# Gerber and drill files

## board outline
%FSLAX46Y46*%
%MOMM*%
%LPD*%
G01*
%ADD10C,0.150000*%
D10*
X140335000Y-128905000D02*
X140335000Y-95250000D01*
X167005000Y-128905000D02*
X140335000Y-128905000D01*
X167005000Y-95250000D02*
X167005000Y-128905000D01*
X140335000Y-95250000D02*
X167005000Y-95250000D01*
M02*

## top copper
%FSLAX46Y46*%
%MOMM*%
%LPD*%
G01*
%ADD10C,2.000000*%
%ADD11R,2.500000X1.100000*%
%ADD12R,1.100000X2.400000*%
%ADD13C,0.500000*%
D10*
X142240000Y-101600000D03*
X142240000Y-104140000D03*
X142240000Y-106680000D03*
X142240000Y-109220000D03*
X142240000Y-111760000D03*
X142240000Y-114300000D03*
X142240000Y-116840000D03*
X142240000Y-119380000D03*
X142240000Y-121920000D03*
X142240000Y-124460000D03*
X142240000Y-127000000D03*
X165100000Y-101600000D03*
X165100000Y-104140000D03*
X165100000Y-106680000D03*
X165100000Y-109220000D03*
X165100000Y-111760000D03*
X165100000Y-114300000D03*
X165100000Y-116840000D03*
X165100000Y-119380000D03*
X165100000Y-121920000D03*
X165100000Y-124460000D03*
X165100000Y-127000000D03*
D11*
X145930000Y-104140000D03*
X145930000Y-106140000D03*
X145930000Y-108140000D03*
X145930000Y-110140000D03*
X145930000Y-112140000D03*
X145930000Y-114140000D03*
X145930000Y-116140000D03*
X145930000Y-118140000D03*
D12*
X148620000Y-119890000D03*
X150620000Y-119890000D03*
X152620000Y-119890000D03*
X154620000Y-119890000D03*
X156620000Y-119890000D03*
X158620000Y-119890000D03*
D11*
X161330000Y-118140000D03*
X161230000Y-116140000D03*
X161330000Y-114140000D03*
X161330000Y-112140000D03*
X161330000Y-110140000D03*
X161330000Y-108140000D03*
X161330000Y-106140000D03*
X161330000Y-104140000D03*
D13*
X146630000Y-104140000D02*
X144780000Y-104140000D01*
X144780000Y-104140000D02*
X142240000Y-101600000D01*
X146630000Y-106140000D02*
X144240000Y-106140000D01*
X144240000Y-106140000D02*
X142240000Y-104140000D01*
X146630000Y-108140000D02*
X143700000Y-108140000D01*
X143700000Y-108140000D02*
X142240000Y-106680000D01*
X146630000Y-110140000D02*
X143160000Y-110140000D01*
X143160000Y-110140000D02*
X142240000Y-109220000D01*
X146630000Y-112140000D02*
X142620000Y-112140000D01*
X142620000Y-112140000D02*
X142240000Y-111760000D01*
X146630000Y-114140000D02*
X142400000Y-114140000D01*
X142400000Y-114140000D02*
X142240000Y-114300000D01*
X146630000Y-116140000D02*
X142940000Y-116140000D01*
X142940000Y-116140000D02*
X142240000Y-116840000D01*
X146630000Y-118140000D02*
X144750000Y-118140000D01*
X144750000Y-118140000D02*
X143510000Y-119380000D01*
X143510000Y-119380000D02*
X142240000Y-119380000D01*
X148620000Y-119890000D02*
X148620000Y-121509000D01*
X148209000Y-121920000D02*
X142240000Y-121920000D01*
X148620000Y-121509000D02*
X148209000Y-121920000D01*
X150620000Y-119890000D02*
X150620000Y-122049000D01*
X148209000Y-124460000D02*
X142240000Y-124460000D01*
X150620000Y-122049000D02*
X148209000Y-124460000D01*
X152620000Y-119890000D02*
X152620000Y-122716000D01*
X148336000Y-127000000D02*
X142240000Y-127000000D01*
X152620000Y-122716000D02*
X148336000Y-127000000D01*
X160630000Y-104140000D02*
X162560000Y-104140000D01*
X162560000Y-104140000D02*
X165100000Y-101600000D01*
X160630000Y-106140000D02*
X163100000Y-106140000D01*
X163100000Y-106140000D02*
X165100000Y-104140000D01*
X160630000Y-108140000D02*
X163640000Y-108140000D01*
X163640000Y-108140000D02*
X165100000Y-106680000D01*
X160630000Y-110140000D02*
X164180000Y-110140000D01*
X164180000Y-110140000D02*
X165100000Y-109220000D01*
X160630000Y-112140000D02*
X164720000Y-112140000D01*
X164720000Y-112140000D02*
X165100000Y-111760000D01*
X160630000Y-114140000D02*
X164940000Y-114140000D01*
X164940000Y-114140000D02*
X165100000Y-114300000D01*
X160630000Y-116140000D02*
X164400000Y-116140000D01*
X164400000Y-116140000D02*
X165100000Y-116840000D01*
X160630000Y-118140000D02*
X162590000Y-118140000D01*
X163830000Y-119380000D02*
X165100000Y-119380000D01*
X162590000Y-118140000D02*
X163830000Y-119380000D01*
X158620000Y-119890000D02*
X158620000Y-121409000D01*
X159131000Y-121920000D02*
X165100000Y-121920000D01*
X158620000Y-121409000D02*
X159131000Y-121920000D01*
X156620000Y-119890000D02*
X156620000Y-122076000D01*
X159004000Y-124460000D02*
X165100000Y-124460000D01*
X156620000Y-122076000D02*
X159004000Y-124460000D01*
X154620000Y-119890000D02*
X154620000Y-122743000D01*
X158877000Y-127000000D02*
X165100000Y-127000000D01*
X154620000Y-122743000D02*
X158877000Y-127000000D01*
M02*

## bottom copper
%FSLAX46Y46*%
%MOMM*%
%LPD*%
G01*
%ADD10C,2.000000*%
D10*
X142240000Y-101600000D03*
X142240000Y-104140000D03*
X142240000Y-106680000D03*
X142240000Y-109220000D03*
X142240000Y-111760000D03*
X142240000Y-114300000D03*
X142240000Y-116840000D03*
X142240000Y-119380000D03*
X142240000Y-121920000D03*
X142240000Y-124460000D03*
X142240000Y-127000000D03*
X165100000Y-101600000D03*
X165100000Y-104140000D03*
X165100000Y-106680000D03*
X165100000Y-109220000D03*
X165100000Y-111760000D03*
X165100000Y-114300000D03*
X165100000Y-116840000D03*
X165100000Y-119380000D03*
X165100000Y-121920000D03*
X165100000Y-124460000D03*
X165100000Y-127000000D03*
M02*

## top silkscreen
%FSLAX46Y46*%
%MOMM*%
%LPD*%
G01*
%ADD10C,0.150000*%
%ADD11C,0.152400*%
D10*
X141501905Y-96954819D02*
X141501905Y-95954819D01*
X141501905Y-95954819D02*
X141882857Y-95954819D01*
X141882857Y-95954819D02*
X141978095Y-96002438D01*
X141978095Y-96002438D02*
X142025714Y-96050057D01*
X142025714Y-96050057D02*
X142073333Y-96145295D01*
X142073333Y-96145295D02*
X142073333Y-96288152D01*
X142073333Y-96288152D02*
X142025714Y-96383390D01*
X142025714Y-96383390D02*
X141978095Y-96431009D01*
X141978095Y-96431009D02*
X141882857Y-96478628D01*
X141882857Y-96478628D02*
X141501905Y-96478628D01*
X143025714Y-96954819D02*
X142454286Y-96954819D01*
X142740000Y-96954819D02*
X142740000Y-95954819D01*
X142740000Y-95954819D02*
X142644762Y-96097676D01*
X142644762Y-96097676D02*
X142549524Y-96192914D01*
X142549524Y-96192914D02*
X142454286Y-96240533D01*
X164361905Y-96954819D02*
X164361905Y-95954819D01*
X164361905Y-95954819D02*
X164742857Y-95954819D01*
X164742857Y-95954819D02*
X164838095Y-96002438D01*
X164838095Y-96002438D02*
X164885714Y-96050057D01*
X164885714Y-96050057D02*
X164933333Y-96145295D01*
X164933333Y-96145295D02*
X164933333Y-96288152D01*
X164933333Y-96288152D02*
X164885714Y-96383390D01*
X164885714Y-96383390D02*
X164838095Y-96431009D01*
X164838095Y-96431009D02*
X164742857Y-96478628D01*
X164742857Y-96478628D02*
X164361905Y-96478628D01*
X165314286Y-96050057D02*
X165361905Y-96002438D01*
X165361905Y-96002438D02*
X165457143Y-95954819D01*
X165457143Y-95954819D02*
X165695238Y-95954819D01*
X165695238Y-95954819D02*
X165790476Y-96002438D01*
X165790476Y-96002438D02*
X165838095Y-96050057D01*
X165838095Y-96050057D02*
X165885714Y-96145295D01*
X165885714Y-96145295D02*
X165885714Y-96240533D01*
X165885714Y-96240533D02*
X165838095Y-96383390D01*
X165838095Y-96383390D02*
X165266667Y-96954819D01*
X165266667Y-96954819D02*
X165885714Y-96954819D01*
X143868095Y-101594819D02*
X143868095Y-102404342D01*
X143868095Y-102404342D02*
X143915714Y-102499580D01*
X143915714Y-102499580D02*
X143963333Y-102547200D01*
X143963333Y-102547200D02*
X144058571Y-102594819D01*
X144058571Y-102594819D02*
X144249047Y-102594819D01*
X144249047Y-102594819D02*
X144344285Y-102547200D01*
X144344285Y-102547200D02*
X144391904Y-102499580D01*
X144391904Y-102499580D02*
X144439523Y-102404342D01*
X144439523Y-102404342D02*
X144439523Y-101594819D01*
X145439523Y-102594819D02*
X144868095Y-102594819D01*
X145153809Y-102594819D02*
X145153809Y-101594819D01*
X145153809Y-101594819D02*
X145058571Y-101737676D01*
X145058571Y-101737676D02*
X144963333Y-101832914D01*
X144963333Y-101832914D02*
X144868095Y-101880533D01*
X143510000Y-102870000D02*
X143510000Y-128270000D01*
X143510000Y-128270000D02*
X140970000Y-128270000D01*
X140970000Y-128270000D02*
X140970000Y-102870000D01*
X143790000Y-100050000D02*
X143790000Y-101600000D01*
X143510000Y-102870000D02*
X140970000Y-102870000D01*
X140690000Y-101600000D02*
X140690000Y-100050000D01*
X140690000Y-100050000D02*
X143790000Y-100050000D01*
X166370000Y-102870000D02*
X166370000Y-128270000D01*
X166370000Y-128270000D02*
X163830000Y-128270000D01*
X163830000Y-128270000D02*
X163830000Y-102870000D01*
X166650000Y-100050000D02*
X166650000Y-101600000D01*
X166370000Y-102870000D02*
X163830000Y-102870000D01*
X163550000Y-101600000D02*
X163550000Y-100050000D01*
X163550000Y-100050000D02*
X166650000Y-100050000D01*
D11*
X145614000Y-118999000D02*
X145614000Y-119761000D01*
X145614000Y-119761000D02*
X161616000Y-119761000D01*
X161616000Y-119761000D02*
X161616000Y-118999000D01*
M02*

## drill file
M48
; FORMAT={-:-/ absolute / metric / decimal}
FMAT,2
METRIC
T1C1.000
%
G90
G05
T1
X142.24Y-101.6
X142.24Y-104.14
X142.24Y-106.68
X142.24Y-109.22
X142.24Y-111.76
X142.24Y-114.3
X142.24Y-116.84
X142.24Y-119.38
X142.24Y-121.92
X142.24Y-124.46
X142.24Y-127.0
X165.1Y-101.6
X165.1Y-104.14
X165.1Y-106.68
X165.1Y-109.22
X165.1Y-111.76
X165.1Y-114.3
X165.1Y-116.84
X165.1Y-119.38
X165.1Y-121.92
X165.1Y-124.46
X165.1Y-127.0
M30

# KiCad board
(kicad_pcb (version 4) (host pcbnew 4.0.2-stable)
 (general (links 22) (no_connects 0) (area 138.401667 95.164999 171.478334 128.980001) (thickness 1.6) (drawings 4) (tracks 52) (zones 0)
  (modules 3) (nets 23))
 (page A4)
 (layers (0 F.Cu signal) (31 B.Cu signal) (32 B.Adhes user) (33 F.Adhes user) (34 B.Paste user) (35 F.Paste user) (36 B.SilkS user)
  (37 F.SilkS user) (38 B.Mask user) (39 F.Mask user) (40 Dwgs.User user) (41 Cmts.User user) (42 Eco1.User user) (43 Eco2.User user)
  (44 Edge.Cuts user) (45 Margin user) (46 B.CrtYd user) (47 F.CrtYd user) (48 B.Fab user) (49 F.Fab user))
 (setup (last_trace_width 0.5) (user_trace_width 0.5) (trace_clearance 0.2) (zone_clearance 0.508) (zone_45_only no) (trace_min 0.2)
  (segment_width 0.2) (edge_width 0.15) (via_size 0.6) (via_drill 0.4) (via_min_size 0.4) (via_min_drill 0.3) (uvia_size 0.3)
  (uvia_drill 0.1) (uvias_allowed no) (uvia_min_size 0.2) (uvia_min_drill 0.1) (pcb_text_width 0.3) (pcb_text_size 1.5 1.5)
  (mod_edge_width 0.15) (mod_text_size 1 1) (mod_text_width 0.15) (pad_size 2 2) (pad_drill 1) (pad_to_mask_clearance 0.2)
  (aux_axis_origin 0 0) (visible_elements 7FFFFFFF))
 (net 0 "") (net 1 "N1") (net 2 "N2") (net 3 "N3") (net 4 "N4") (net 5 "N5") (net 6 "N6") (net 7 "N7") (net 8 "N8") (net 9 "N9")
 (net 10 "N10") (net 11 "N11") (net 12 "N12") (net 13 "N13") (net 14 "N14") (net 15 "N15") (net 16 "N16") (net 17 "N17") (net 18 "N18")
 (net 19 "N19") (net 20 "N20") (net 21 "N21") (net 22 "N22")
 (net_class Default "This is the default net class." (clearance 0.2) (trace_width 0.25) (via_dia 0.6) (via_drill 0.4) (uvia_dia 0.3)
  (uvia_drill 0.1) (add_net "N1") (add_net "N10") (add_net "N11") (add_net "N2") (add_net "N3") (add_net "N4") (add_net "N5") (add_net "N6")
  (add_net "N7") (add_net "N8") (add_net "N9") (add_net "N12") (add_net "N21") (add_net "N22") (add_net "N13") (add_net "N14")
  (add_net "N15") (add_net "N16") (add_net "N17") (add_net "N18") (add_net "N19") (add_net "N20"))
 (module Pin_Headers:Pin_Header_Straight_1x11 (layer F.Cu) (at 142.24 101.6)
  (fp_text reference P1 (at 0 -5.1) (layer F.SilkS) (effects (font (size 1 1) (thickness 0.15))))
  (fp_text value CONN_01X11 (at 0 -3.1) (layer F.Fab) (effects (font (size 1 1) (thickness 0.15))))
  (fp_line (start 1.27 1.27) (end 1.27 26.67) (layer F.SilkS) (width 0.15))
  (fp_line (start 1.27 26.67) (end -1.27 26.67) (layer F.SilkS) (width 0.15))
  (fp_line (start -1.27 26.67) (end -1.27 1.27) (layer F.SilkS) (width 0.15))
  (fp_line (start 1.55 -1.55) (end 1.55 0) (layer F.SilkS) (width 0.15))
  (fp_line (start 1.27 1.27) (end -1.27 1.27) (layer F.SilkS) (width 0.15))
  (fp_line (start -1.55 0) (end -1.55 -1.55) (layer F.SilkS) (width 0.15))
  (fp_line (start -1.55 -1.55) (end 1.55 -1.55) (layer F.SilkS) (width 0.15))
  (pad 1 thru_hole circle (at 0 0) (size 2 2) (drill 1) (layers *.Cu *.Mask) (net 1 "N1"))
  (pad 2 thru_hole circle (at 0 2.54) (size 2 2) (drill 1) (layers *.Cu *.Mask) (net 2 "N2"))
  (pad 3 thru_hole circle (at 0 5.08) (size 2 2) (drill 1) (layers *.Cu *.Mask) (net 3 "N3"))
  (pad 4 thru_hole circle (at 0 7.62) (size 2 2) (drill 1) (layers *.Cu *.Mask) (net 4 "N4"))
  (pad 5 thru_hole circle (at 0 10.16) (size 2 2) (drill 1) (layers *.Cu *.Mask) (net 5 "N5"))
  (pad 6 thru_hole circle (at 0 12.7) (size 2 2) (drill 1) (layers *.Cu *.Mask) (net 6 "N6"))
  (pad 7 thru_hole circle (at 0 15.24) (size 2 2) (drill 1) (layers *.Cu *.Mask) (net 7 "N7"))
  (pad 8 thru_hole circle (at 0 17.78) (size 2 2) (drill 1) (layers *.Cu *.Mask) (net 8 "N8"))
  (pad 9 thru_hole circle (at 0 20.32) (size 2 2) (drill 1) (layers *.Cu *.Mask) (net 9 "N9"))
  (pad 10 thru_hole circle (at 0 22.86) (size 2 2) (drill 1) (layers *.Cu *.Mask) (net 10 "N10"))
  (pad 11 thru_hole circle (at 0 25.4) (size 2 2) (drill 1) (layers *.Cu *.Mask) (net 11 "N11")))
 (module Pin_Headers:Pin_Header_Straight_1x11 (layer F.Cu) (at 165.1 101.6)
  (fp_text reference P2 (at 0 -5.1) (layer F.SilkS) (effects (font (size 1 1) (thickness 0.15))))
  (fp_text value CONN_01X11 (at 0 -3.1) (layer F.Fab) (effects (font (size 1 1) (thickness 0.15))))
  (fp_line (start 1.27 1.27) (end 1.27 26.67) (layer F.SilkS) (width 0.15))
  (fp_line (start 1.27 26.67) (end -1.27 26.67) (layer F.SilkS) (width 0.15))
  (fp_line (start -1.27 26.67) (end -1.27 1.27) (layer F.SilkS) (width 0.15))
  (fp_line (start 1.55 -1.55) (end 1.55 0) (layer F.SilkS) (width 0.15))
  (fp_line (start 1.27 1.27) (end -1.27 1.27) (layer F.SilkS) (width 0.15))
  (fp_line (start -1.55 0) (end -1.55 -1.55) (layer F.SilkS) (width 0.15))
  (fp_line (start -1.55 -1.55) (end 1.55 -1.55) (layer F.SilkS) (width 0.15))
  (pad 1 thru_hole circle (at 0 0) (size 2 2) (drill 1) (layers *.Cu *.Mask) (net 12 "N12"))
  (pad 2 thru_hole circle (at 0 2.54) (size 2 2) (drill 1) (layers *.Cu *.Mask) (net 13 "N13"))
  (pad 3 thru_hole circle (at 0 5.08) (size 2 2) (drill 1) (layers *.Cu *.Mask) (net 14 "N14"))
  (pad 4 thru_hole circle (at 0 7.62) (size 2 2) (drill 1) (layers *.Cu *.Mask) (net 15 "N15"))
  (pad 5 thru_hole circle (at 0 10.16) (size 2 2) (drill 1) (layers *.Cu *.Mask) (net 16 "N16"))
  (pad 6 thru_hole circle (at 0 12.7) (size 2 2) (drill 1) (layers *.Cu *.Mask) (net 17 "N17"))
  (pad 7 thru_hole circle (at 0 15.24) (size 2 2) (drill 1) (layers *.Cu *.Mask) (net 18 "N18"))
  (pad 8 thru_hole circle (at 0 17.78) (size 2 2) (drill 1) (layers *.Cu *.Mask) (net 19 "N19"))
  (pad 9 thru_hole circle (at 0 20.32) (size 2 2) (drill 1) (layers *.Cu *.Mask) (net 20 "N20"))
  (pad 10 thru_hole circle (at 0 22.86) (size 2 2) (drill 1) (layers *.Cu *.Mask) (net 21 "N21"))
  (pad 11 thru_hole circle (at 0 25.4) (size 2 2) (drill 1) (layers *.Cu *.Mask) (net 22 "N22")))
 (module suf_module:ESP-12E (layer F.Cu) (at 146.63 104.14)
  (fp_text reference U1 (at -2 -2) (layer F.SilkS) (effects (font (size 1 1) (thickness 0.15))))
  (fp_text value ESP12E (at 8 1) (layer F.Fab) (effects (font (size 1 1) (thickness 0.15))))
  (fp_line (start -1.016 14.859) (end -1.016 15.621) (layer F.SilkS) (width 0.1524))
  (fp_line (start -1.016 15.621) (end 14.986 15.621) (layer F.SilkS) (width 0.1524))
  (fp_line (start 14.986 15.621) (end 14.986 14.859) (layer F.SilkS) (width 0.1524))
  (pad 1 smd rect (at 0 0) (size 2.5 1.1) (drill (offset -0.7 0)) (layers F.Cu F.Paste F.Mask) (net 1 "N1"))
  (pad 2 smd rect (at 0 2) (size 2.5 1.1) (drill (offset -0.7 0)) (layers F.Cu F.Paste F.Mask) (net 2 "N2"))
  (pad 3 smd rect (at 0 4) (size 2.5 1.1) (drill (offset -0.7 0)) (layers F.Cu F.Paste F.Mask) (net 3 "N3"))
  (pad 4 smd rect (at 0 6) (size 2.5 1.1) (drill (offset -0.7 0)) (layers F.Cu F.Paste F.Mask) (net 4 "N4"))
  (pad 5 smd rect (at 0 8) (size 2.5 1.1) (drill (offset -0.7 0)) (layers F.Cu F.Paste F.Mask) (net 5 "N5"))
  (pad 6 smd rect (at 0 10) (size 2.5 1.1) (drill (offset -0.7 0)) (layers F.Cu F.Paste F.Mask) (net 6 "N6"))
  (pad 7 smd rect (at 0 12) (size 2.5 1.1) (drill (offset -0.7 0)) (layers F.Cu F.Paste F.Mask) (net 7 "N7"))
  (pad 8 smd rect (at 0 14) (size 2.5 1.1) (drill (offset -0.7 0)) (layers F.Cu F.Paste F.Mask) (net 8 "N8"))
  (pad 17 smd rect (at 1.99 15.75 90) (size 2.4 1.1) (layers F.Cu F.Paste F.Mask) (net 9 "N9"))
  (pad 18 smd rect (at 3.99 15.75 90) (size 2.4 1.1) (layers F.Cu F.Paste F.Mask) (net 10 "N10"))
  (pad 19 smd rect (at 5.99 15.75 90) (size 2.4 1.1) (layers F.Cu F.Paste F.Mask) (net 11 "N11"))
  (pad 20 smd rect (at 7.99 15.75 90) (size 2.4 1.1) (layers F.Cu F.Paste F.Mask) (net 22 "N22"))
  (pad 21 smd rect (at 9.99 15.75 90) (size 2.4 1.1) (layers F.Cu F.Paste F.Mask) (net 21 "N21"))
  (pad 22 smd rect (at 11.99 15.75 90) (size 2.4 1.1) (layers F.Cu F.Paste F.Mask) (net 20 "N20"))
  (pad 9 smd rect (at 14 14) (size 2.5 1.1) (drill (offset 0.7 0)) (layers F.Cu F.Paste F.Mask) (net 19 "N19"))
  (pad 10 smd rect (at 14 12) (size 2.5 1.1) (drill (offset 0.6 0)) (layers F.Cu F.Paste F.Mask) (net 18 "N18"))
  (pad 11 smd rect (at 14 10) (size 2.5 1.1) (drill (offset 0.7 0)) (layers F.Cu F.Paste F.Mask) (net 17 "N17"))
  (pad 12 smd rect (at 14 8) (size 2.5 1.1) (drill (offset 0.7 0)) (layers F.Cu F.Paste F.Mask) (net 16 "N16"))
  (pad 13 smd rect (at 14 6) (size 2.5 1.1) (drill (offset 0.7 0)) (layers F.Cu F.Paste F.Mask) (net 15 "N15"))
  (pad 14 smd rect (at 14 4) (size 2.5 1.1) (drill (offset 0.7 0)) (layers F.Cu F.Paste F.Mask) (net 14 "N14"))
  (pad 15 smd rect (at 14 2) (size 2.5 1.1) (drill (offset 0.7 0)) (layers F.Cu F.Paste F.Mask) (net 13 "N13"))
  (pad 16 smd rect (at 14 0) (size 2.5 1.1) (drill (offset 0.7 0)) (layers F.Cu F.Paste F.Mask) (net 12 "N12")))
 (gr_line (start 140.335 128.905) (end 140.335 95.25) (angle 90) (layer Edge.Cuts) (width 0.15))
 (gr_line (start 167.005 128.905) (end 140.335 128.905) (angle 90) (layer Edge.Cuts) (width 0.15))
 (gr_line (start 167.005 95.25) (end 167.005 128.905) (angle 90) (layer Edge.Cuts) (width 0.15))
 (gr_line (start 140.335 95.25) (end 167.005 95.25) (angle 90) (layer Edge.Cuts) (width 0.15))
 (segment (start 146.63 104.14) (end 144.78 104.14) (width 0.5) (layer F.Cu) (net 1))
 (segment (start 144.78 104.14) (end 142.24 101.6) (width 0.5) (layer F.Cu) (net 1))
 (segment (start 146.63 106.14) (end 144.24 106.14) (width 0.5) (layer F.Cu) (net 2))
 (segment (start 144.24 106.14) (end 142.24 104.14) (width 0.5) (layer F.Cu) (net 2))
 (segment (start 146.63 108.14) (end 143.7 108.14) (width 0.5) (layer F.Cu) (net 3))
 (segment (start 143.7 108.14) (end 142.24 106.68) (width 0.5) (layer F.Cu) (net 3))
 (segment (start 146.63 110.14) (end 143.16 110.14) (width 0.5) (layer F.Cu) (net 4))
 (segment (start 143.16 110.14) (end 142.24 109.22) (width 0.5) (layer F.Cu) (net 4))
 (segment (start 146.63 112.14) (end 142.62 112.14) (width 0.5) (layer F.Cu) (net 5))
 (segment (start 142.62 112.14) (end 142.24 111.76) (width 0.5) (layer F.Cu) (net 5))
 (segment (start 146.63 114.14) (end 142.4 114.14) (width 0.5) (layer F.Cu) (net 6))
 (segment (start 142.4 114.14) (end 142.24 114.3) (width 0.5) (layer F.Cu) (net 6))
 (segment (start 146.63 116.14) (end 142.94 116.14) (width 0.5) (layer F.Cu) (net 7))
 (segment (start 142.94 116.14) (end 142.24 116.84) (width 0.5) (layer F.Cu) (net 7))
 (segment (start 146.63 118.14) (end 144.75 118.14) (width 0.5) (layer F.Cu) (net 8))
 (segment (start 144.75 118.14) (end 143.51 119.38) (width 0.5) (layer F.Cu) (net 8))
 (segment (start 143.51 119.38) (end 142.24 119.38) (width 0.5) (layer F.Cu) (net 8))
 (segment (start 148.62 119.89) (end 148.62 121.509) (width 0.5) (layer F.Cu) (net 9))
 (segment (start 148.209 121.92) (end 142.24 121.92) (width 0.5) (layer F.Cu) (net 9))
 (segment (start 148.62 121.509) (end 148.209 121.92) (width 0.5) (layer F.Cu) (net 9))
 (segment (start 150.62 119.89) (end 150.62 122.049) (width 0.5) (layer F.Cu) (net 10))
 (segment (start 148.209 124.46) (end 142.24 124.46) (width 0.5) (layer F.Cu) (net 10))
 (segment (start 150.62 122.049) (end 148.209 124.46) (width 0.5) (layer F.Cu) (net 10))
 (segment (start 152.62 119.89) (end 152.62 122.716) (width 0.5) (layer F.Cu) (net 11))
 (segment (start 148.336 127) (end 142.24 127) (width 0.5) (layer F.Cu) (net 11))
 (segment (start 152.62 122.716) (end 148.336 127) (width 0.5) (layer F.Cu) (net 11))
 (segment (start 160.63 104.14) (end 162.56 104.14) (width 0.5) (layer F.Cu) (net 12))
 (segment (start 162.56 104.14) (end 165.1 101.6) (width 0.5) (layer F.Cu) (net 12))
 (segment (start 160.63 106.14) (end 163.1 106.14) (width 0.5) (layer F.Cu) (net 13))
 (segment (start 163.1 106.14) (end 165.1 104.14) (width 0.5) (layer F.Cu) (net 13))
 (segment (start 160.63 108.14) (end 163.64 108.14) (width 0.5) (layer F.Cu) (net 14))
 (segment (start 163.64 108.14) (end 165.1 106.68) (width 0.5) (layer F.Cu) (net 14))
 (segment (start 160.63 110.14) (end 164.18 110.14) (width 0.5) (layer F.Cu) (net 15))
 (segment (start 164.18 110.14) (end 165.1 109.22) (width 0.5) (layer F.Cu) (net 15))
 (segment (start 160.63 112.14) (end 164.72 112.14) (width 0.5) (layer F.Cu) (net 16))
 (segment (start 164.72 112.14) (end 165.1 111.76) (width 0.5) (layer F.Cu) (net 16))
 (segment (start 160.63 114.14) (end 164.94 114.14) (width 0.5) (layer F.Cu) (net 17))
 (segment (start 164.94 114.14) (end 165.1 114.3) (width 0.5) (layer F.Cu) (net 17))
 (segment (start 160.63 116.14) (end 164.4 116.14) (width 0.5) (layer F.Cu) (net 18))
 (segment (start 164.4 116.14) (end 165.1 116.84) (width 0.5) (layer F.Cu) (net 18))
 (segment (start 160.63 118.14) (end 162.59 118.14) (width 0.5) (layer F.Cu) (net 19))
 (segment (start 163.83 119.38) (end 165.1 119.38) (width 0.5) (layer F.Cu) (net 19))
 (segment (start 162.59 118.14) (end 163.83 119.38) (width 0.5) (layer F.Cu) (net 19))
 (segment (start 158.62 119.89) (end 158.62 121.409) (width 0.5) (layer F.Cu) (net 20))
 (segment (start 159.131 121.92) (end 165.1 121.92) (width 0.5) (layer F.Cu) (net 20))
 (segment (start 158.62 121.409) (end 159.131 121.92) (width 0.5) (layer F.Cu) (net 20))
 (segment (start 156.62 119.89) (end 156.62 122.076) (width 0.5) (layer F.Cu) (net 21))
 (segment (start 159.004 124.46) (end 165.1 124.46) (width 0.5) (layer F.Cu) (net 21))
 (segment (start 156.62 122.076) (end 159.004 124.46) (width 0.5) (layer F.Cu) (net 21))
 (segment (start 154.62 119.89) (end 154.62 122.743) (width 0.5) (layer F.Cu) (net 22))
 (segment (start 158.877 127) (end 165.1 127) (width 0.5) (layer F.Cu) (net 22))
 (segment (start 154.62 122.743) (end 158.877 127) (width 0.5) (layer F.Cu) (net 22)))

